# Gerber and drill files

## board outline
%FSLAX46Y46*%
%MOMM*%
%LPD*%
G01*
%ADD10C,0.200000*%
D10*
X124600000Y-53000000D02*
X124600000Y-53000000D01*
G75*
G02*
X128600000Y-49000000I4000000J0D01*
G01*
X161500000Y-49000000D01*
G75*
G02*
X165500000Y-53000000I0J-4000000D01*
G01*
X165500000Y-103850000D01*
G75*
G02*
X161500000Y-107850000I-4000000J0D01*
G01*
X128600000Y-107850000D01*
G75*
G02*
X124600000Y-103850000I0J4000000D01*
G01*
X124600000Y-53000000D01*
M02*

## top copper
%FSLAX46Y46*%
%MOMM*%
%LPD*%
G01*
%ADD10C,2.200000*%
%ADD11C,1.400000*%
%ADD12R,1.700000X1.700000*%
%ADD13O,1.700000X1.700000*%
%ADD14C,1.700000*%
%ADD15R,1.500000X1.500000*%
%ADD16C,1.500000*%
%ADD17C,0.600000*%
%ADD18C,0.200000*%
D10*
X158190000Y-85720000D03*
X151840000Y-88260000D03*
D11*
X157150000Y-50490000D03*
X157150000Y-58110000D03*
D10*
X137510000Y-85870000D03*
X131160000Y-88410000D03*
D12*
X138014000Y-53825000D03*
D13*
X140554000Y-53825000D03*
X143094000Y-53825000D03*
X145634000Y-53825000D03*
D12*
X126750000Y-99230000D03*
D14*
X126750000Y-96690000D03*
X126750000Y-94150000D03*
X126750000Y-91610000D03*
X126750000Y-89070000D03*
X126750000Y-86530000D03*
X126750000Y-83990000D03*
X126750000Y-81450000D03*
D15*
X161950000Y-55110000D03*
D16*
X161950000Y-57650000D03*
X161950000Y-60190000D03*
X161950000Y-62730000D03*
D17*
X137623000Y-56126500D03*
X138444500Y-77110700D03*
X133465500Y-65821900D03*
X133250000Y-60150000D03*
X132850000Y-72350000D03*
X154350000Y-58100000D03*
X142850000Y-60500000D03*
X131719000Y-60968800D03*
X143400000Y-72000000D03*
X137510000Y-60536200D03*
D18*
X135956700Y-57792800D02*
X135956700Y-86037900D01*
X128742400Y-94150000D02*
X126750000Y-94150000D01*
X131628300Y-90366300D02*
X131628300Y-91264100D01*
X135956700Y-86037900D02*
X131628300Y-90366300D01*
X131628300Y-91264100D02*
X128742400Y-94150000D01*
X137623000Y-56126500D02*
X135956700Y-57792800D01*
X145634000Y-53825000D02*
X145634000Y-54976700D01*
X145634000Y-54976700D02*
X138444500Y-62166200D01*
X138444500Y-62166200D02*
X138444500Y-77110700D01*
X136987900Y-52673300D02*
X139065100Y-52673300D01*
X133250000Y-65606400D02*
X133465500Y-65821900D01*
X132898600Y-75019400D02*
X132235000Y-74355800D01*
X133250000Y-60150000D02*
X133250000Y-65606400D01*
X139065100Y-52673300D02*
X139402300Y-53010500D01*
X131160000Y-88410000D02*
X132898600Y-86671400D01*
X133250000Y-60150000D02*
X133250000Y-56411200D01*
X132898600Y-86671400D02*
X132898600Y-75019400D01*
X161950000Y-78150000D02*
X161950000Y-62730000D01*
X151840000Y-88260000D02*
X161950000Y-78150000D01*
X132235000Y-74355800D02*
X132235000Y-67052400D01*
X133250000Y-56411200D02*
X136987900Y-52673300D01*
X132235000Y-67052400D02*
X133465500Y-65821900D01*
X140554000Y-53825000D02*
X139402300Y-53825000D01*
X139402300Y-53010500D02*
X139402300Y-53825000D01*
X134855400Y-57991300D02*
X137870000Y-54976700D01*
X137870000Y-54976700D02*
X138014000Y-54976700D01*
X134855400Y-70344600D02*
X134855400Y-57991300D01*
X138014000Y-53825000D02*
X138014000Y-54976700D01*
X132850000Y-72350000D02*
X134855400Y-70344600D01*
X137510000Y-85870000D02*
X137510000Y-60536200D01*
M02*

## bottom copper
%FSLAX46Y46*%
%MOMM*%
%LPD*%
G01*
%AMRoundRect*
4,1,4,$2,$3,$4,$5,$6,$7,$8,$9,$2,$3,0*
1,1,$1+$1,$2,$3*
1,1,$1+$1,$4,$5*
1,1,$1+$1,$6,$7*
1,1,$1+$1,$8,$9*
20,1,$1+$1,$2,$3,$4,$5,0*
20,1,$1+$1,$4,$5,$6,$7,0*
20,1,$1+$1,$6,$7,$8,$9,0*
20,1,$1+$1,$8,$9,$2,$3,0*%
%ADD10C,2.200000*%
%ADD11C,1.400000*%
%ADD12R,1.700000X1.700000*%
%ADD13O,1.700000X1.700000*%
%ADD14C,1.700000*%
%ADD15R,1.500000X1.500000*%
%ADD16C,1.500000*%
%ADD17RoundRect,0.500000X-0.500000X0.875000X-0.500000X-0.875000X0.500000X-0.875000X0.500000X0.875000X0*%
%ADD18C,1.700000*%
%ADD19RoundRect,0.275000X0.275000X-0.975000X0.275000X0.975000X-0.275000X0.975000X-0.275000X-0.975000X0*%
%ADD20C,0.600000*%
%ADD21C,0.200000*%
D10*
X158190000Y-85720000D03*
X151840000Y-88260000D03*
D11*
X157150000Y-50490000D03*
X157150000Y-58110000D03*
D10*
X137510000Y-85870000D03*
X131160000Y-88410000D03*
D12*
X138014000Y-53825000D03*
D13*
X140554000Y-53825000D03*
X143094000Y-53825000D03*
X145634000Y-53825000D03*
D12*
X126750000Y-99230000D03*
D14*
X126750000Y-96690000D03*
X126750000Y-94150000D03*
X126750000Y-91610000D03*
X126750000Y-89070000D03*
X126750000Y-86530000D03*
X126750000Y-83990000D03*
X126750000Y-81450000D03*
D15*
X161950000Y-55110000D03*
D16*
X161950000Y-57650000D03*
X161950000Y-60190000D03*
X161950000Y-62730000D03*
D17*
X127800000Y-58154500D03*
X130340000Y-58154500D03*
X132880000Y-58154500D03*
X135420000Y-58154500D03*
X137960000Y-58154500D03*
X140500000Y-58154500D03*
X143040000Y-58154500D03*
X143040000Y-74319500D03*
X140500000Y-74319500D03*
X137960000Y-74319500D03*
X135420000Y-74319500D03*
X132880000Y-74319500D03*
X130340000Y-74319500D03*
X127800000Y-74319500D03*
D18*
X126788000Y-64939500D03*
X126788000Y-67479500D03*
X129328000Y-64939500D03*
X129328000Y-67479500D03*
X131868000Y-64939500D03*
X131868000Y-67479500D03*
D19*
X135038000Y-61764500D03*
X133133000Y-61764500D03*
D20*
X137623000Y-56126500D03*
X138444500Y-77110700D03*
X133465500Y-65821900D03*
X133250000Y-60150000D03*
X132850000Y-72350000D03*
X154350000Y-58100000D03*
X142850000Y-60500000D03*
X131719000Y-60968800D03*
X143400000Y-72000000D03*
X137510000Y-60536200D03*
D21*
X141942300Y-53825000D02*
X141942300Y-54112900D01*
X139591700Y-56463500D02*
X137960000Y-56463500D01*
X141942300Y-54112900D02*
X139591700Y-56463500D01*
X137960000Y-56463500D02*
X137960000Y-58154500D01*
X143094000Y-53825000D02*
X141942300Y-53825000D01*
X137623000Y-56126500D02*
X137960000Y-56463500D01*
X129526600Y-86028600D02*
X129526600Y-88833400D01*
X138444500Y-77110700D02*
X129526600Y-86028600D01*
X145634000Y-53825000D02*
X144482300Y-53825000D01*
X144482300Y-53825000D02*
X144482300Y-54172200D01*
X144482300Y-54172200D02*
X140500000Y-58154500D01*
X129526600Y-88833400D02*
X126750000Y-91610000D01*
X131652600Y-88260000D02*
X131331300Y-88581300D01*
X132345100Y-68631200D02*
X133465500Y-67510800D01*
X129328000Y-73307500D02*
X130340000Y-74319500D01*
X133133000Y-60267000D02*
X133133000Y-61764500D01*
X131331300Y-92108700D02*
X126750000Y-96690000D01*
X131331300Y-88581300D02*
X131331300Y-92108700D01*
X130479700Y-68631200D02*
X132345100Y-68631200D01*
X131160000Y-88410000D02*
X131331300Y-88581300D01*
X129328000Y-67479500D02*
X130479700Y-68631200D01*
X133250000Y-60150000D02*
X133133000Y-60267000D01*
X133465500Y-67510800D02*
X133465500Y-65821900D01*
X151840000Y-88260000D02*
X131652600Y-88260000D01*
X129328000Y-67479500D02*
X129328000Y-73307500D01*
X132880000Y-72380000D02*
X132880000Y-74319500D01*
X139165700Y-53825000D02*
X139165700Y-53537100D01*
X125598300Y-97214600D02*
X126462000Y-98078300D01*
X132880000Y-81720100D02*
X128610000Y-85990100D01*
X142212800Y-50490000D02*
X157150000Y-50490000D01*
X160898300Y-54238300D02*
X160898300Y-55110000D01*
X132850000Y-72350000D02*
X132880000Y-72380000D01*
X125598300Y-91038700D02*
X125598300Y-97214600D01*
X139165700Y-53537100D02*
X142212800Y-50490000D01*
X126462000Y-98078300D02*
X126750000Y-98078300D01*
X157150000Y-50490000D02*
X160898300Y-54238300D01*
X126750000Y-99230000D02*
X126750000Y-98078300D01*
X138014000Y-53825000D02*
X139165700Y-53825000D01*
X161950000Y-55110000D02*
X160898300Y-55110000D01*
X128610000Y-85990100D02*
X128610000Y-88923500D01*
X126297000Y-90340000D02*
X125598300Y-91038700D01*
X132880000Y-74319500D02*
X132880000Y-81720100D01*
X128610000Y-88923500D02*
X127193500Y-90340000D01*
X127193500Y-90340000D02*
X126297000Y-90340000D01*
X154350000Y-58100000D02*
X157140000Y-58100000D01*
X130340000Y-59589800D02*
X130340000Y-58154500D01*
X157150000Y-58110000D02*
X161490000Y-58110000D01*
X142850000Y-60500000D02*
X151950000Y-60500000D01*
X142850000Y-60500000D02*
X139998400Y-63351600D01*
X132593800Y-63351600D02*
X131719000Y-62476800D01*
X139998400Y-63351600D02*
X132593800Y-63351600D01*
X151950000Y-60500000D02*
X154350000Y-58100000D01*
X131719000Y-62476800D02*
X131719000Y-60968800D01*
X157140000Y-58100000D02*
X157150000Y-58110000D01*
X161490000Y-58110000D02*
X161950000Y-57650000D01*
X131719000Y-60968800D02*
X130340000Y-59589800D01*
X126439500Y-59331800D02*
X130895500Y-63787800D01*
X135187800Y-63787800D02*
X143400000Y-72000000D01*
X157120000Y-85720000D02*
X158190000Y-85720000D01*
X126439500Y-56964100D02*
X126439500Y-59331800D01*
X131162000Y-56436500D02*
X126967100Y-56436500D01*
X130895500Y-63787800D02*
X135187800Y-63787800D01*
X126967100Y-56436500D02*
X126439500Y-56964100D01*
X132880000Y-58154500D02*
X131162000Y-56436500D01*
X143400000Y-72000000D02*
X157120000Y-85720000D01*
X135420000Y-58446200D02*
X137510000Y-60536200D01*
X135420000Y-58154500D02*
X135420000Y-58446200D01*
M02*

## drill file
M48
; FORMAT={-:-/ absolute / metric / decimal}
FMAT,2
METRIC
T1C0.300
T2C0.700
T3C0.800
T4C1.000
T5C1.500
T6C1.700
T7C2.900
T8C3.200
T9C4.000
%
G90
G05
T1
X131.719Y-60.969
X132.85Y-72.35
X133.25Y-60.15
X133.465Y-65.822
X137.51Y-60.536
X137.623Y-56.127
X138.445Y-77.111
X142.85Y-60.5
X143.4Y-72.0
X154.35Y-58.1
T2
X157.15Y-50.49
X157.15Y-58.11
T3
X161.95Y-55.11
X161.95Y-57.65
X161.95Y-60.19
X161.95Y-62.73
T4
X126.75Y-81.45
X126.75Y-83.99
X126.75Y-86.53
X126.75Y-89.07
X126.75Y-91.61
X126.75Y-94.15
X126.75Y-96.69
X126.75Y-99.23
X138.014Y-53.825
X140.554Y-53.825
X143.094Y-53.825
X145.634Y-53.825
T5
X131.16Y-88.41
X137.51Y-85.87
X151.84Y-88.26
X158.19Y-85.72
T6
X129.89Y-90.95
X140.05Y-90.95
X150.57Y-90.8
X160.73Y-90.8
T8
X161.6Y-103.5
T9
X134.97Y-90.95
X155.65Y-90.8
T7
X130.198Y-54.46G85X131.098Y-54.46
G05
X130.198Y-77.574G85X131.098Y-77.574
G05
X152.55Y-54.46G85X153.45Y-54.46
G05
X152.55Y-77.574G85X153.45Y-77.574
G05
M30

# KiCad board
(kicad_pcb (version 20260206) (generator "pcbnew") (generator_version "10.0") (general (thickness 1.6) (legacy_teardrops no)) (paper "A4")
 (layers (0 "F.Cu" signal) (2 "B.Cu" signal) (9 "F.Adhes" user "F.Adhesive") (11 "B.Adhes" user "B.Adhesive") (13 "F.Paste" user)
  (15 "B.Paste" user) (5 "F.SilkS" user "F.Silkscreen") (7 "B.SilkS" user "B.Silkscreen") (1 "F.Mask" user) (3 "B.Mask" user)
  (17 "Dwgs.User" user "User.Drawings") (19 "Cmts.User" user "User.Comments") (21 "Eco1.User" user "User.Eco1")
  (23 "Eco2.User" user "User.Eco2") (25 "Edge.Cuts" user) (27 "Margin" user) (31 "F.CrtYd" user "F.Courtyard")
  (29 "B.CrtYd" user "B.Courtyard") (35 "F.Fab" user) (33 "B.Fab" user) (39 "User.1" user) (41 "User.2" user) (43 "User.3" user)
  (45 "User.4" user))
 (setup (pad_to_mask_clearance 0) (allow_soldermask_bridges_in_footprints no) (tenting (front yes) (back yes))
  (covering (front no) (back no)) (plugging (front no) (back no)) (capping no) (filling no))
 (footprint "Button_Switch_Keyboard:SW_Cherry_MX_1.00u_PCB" (layer "F.Cu") (at 158.19 85.72)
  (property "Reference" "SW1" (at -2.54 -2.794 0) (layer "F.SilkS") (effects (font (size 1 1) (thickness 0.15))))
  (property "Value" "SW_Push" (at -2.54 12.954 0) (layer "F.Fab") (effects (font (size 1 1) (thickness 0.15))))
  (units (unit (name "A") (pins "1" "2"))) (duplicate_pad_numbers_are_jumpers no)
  (pad "" np_thru_hole circle (at -7.62 5.08) (size 1.7 1.7) (drill 1.7) (layers "*.Cu" "*.Mask"))
  (pad "" np_thru_hole circle (at -2.54 5.08) (size 4 4) (drill 4) (layers "*.Cu" "*.Mask"))
  (pad "" np_thru_hole circle (at 2.54 5.08) (size 1.7 1.7) (drill 1.7) (layers "*.Cu" "*.Mask"))
  (pad "1" thru_hole circle (at 0 0) (size 2.2 2.2) (drill 1.5) (layers "*.Cu" "*.Mask") (remove_unused_layers no) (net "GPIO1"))
  (pad "2" thru_hole circle (at -6.35 2.54) (size 2.2 2.2) (drill 1.5) (layers "*.Cu" "*.Mask") (remove_unused_layers no) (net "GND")))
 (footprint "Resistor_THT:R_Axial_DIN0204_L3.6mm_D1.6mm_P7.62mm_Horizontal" (layer "F.Cu") (at 157.15 50.49 -90)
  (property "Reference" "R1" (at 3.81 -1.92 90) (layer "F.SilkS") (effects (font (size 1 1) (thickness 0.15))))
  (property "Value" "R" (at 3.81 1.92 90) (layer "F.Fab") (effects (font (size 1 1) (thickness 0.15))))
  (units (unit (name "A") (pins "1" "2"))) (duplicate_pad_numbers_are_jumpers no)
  (pad "1" thru_hole circle (at 0 0 270) (size 1.4 1.4) (drill 0.7) (layers "*.Cu" "*.Mask") (remove_unused_layers no) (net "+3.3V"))
  (pad "2" thru_hole circle (at 7.62 0 270) (size 1.4 1.4) (drill 0.7) (layers "*.Cu" "*.Mask") (remove_unused_layers no) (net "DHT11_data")))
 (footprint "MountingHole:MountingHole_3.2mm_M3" (layer "F.Cu") (at 161.6 103.5)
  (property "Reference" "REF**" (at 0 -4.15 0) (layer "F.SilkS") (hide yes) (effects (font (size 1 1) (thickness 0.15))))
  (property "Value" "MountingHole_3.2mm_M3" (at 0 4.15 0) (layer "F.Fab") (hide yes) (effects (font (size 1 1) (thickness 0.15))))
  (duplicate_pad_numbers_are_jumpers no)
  (pad "" np_thru_hole circle (at 0 0) (size 3.2 3.2) (drill 3.2) (layers "*.Cu" "*.Mask")))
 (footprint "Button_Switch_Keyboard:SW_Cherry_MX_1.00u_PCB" (layer "F.Cu") (at 137.51 85.87)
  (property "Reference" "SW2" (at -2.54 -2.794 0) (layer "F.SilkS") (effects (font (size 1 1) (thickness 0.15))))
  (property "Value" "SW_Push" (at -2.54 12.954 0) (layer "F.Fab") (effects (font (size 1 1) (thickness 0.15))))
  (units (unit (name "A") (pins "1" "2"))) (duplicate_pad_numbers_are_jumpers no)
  (pad "" np_thru_hole circle (at -7.62 5.08) (size 1.7 1.7) (drill 1.7) (layers "*.Cu" "*.Mask"))
  (pad "" np_thru_hole circle (at -2.54 5.08) (size 4 4) (drill 4) (layers "*.Cu" "*.Mask"))
  (pad "" np_thru_hole circle (at 2.54 5.08) (size 1.7 1.7) (drill 1.7) (layers "*.Cu" "*.Mask"))
  (pad "1" thru_hole circle (at 0 0) (size 2.2 2.2) (drill 1.5) (layers "*.Cu" "*.Mask") (remove_unused_layers no) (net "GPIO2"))
  (pad "2" thru_hole circle (at -6.35 2.54) (size 2.2 2.2) (drill 1.5) (layers "*.Cu" "*.Mask") (remove_unused_layers no) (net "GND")))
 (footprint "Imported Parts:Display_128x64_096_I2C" (layer "F.Cu") (at 141.824 53.825)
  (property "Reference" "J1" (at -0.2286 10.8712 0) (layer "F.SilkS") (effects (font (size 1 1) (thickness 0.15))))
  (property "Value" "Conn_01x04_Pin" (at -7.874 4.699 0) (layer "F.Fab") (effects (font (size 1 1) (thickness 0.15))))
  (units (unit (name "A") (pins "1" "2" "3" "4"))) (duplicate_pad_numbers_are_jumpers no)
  (pad "" np_thru_hole oval (at -11.176 0.635) (size 3.8 2.9) (drill oval 3.8 2.9) (layers "*.Cu" "*.Mask"))
  (pad "" np_thru_hole oval (at -11.176 23.749) (size 3.8 2.9) (drill oval 3.8 2.9) (layers "*.Cu" "*.Mask"))
  (pad "" np_thru_hole oval (at 11.176 0.635) (size 3.8 2.9) (drill oval 3.8 2.9) (layers "*.Cu" "*.Mask"))
  (pad "" np_thru_hole oval (at 11.176 23.749) (size 3.8 2.9) (drill oval 3.8 2.9) (layers "*.Cu" "*.Mask"))
  (pad "1" thru_hole rect (at -3.81 0 90) (size 1.7 1.7) (drill 1) (layers "*.Cu" "*.Mask") (remove_unused_layers no) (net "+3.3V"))
  (pad "2" thru_hole oval (at -1.27 0 90) (size 1.7 1.7) (drill 1) (layers "*.Cu" "*.Mask") (remove_unused_layers no) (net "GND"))
  (pad "3" thru_hole oval (at 1.27 0 90) (size 1.7 1.7) (drill 1) (layers "*.Cu" "*.Mask") (remove_unused_layers no) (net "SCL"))
  (pad "4" thru_hole oval (at 3.81 0 90) (size 1.7 1.7) (drill 1) (layers "*.Cu" "*.Mask") (remove_unused_layers no) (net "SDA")))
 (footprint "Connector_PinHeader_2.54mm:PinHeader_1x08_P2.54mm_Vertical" (layer "B.Cu") (at 126.75 99.23)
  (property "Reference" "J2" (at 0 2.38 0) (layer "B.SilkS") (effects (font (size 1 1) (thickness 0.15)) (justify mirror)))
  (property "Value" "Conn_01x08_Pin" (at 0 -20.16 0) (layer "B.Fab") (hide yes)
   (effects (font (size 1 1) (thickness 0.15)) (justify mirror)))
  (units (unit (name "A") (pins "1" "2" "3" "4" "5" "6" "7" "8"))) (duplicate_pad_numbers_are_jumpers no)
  (pad "1" thru_hole rect (at 0 0) (size 1.7 1.7) (drill 1) (layers "*.Cu" "*.Mask") (remove_unused_layers no) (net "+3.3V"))
  (pad "2" thru_hole circle (at 0 -2.54) (size 1.7 1.7) (drill 1) (layers "*.Cu" "*.Mask") (remove_unused_layers no) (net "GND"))
  (pad "3" thru_hole circle (at 0 -5.08) (size 1.7 1.7) (drill 1) (layers "*.Cu" "*.Mask") (remove_unused_layers no) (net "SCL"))
  (pad "4" thru_hole circle (at 0 -7.62) (size 1.7 1.7) (drill 1) (layers "*.Cu" "*.Mask") (remove_unused_layers no) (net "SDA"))
  (pad "5" thru_hole circle (at 0 -10.16) (size 1.7 1.7) (drill 1) (layers "*.Cu" "*.Mask") (remove_unused_layers no)
   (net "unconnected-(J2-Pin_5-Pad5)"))
  (pad "6" thru_hole circle (at 0 -12.7) (size 1.7 1.7) (drill 1) (layers "*.Cu" "*.Mask") (remove_unused_layers no)
   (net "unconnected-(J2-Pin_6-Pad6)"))
  (pad "7" thru_hole circle (at 0 -15.24) (size 1.7 1.7) (drill 1) (layers "*.Cu" "*.Mask") (remove_unused_layers no)
   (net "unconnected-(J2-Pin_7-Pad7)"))
  (pad "8" thru_hole circle (at 0 -17.78) (size 1.7 1.7) (drill 1) (layers "*.Cu" "*.Mask") (remove_unused_layers no)
   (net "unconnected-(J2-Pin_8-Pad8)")))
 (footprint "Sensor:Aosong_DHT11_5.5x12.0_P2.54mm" (layer "B.Cu") (at 161.95 55.11 180)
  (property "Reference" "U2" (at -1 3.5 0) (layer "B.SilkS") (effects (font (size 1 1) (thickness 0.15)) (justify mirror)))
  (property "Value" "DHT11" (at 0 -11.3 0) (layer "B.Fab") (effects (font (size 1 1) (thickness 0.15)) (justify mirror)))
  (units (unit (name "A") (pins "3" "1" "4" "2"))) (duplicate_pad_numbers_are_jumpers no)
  (pad "1" thru_hole rect (at 0 0 180) (size 1.5 1.5) (drill 0.8) (layers "*.Cu" "*.Mask") (remove_unused_layers no) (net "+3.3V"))
  (pad "2" thru_hole circle (at 0 -2.54 180) (size 1.5 1.5) (drill 0.8) (layers "*.Cu" "*.Mask") (remove_unused_layers no)
   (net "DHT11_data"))
  (pad "3" thru_hole circle (at 0 -5.08 180) (size 1.5 1.5) (drill 0.8) (layers "*.Cu" "*.Mask") (remove_unused_layers no)
   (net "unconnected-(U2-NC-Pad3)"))
  (pad "4" thru_hole circle (at 0 -7.62 180) (size 1.5 1.5) (drill 0.8) (layers "*.Cu" "*.Mask") (remove_unused_layers no) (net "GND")))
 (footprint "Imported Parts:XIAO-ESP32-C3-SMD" (layer "B.Cu") (at 145.92 57.3195 -90)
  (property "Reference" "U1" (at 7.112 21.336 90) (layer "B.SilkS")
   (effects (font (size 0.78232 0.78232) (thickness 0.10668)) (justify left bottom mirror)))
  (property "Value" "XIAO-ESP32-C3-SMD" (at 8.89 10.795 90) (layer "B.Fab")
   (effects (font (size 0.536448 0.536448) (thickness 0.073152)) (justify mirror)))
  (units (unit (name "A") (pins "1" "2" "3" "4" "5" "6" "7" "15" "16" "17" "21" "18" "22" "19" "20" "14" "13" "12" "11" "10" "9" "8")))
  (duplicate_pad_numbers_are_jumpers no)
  (pad "1" smd roundrect (at 0.835 18.12 270) (size 2.75 2) (layers "B.Cu" "B.Mask" "B.Paste") (roundrect_rratio 0.25)
   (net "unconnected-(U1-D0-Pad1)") (solder_mask_margin 0.0508) (thermal_bridge_angle 45))
  (pad "2" smd roundrect (at 0.835 15.58 270) (size 2.75 2) (layers "B.Cu" "B.Mask" "B.Paste") (roundrect_rratio 0.25) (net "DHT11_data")
   (solder_mask_margin 0.0508) (thermal_bridge_angle 45))
  (pad "3" smd roundrect (at 0.835 13.04 270) (size 2.75 2) (layers "B.Cu" "B.Mask" "B.Paste") (roundrect_rratio 0.25) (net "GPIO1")
   (solder_mask_margin 0.0508) (thermal_bridge_angle 45))
  (pad "4" smd roundrect (at 0.835 10.5 270) (size 2.75 2) (layers "B.Cu" "B.Mask" "B.Paste") (roundrect_rratio 0.25) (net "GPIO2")
   (solder_mask_margin 0.0508) (thermal_bridge_angle 45))
  (pad "5" smd roundrect (at 0.835 7.96 270) (size 2.75 2) (layers "B.Cu" "B.Mask" "B.Paste") (roundrect_rratio 0.25) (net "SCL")
   (solder_mask_margin 0.0508) (thermal_bridge_angle 45))
  (pad "6" smd roundrect (at 0.835 5.42 270) (size 2.75 2) (layers "B.Cu" "B.Mask" "B.Paste") (roundrect_rratio 0.25) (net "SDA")
   (solder_mask_margin 0.0508) (thermal_bridge_angle 45))
  (pad "7" smd roundrect (at 0.835 2.88 270) (size 2.75 2) (layers "B.Cu" "B.Mask" "B.Paste") (roundrect_rratio 0.25)
   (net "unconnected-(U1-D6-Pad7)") (solder_mask_margin 0.0508) (thermal_bridge_angle 45))
  (pad "8" smd roundrect (at 17 2.88 270) (size 2.75 2) (layers "B.Cu" "B.Mask" "B.Paste") (roundrect_rratio 0.25)
   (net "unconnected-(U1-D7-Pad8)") (solder_mask_margin 0.0508) (thermal_bridge_angle 45))
  (pad "9" smd roundrect (at 17 5.42 270) (size 2.75 2) (layers "B.Cu" "B.Mask" "B.Paste") (roundrect_rratio 0.25)
   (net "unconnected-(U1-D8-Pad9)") (solder_mask_margin 0.0508) (thermal_bridge_angle 45))
  (pad "10" smd roundrect (at 17 7.96 270) (size 2.75 2) (layers "B.Cu" "B.Mask" "B.Paste") (roundrect_rratio 0.25)
   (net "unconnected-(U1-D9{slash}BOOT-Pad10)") (solder_mask_margin 0.0508) (thermal_bridge_angle 45))
  (pad "11" smd roundrect (at 17 10.5 270) (size 2.75 2) (layers "B.Cu" "B.Mask" "B.Paste") (roundrect_rratio 0.25)
   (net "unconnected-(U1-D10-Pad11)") (solder_mask_margin 0.0508) (thermal_bridge_angle 45))
  (pad "12" smd roundrect (at 17 13.04 270) (size 2.75 2) (layers "B.Cu" "B.Mask" "B.Paste") (roundrect_rratio 0.25) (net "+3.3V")
   (solder_mask_margin 0.0508) (thermal_bridge_angle 45))
  (pad "13" smd roundrect (at 17 15.58 270) (size 2.75 2) (layers "B.Cu" "B.Mask" "B.Paste") (roundrect_rratio 0.25) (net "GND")
   (solder_mask_margin 0.0508) (thermal_bridge_angle 45))
  (pad "14" smd roundrect (at 17 18.12 270) (size 2.75 2) (layers "B.Cu" "B.Mask" "B.Paste") (roundrect_rratio 0.25) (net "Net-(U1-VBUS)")
   (solder_mask_margin 0.0508) (thermal_bridge_angle 45))
  (pad "15" smd circle (at 7.62 19.132 270) (size 1.7 1.7) (layers "B.Cu" "B.Mask" "B.Paste") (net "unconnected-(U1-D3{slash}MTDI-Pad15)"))
  (pad "16" smd circle (at 10.16 19.132 270) (size 1.7 1.7) (layers "B.Cu" "B.Mask" "B.Paste") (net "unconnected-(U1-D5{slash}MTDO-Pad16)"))
  (pad "17" smd circle (at 7.62 16.592 270) (size 1.7 1.7) (layers "B.Cu" "B.Mask" "B.Paste") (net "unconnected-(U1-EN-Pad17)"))
  (pad "18" smd circle (at 10.16 16.592 270) (size 1.7 1.7) (layers "B.Cu" "B.Mask" "B.Paste") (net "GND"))
  (pad "19" smd circle (at 7.62 14.052 270) (size 1.7 1.7) (layers "B.Cu" "B.Mask" "B.Paste") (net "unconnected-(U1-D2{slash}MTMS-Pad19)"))
  (pad "20" smd circle (at 10.16 14.052 270) (size 1.7 1.7) (layers "B.Cu" "B.Mask" "B.Paste") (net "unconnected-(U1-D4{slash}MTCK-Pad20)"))
  (pad "21" smd roundrect (at 4.445 10.882 90) (size 2.5 1.1) (layers "B.Cu" "B.Mask" "B.Paste") (roundrect_rratio 0.25)
   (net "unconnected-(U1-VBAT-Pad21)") (thermal_bridge_angle 45))
  (pad "22" smd roundrect (at 4.445 12.787 90) (size 2.5 1.1) (layers "B.Cu" "B.Mask" "B.Paste") (roundrect_rratio 0.25) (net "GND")
   (thermal_bridge_angle 45)))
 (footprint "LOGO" (layer "B.Cu") (at 151.821269 66.65 180)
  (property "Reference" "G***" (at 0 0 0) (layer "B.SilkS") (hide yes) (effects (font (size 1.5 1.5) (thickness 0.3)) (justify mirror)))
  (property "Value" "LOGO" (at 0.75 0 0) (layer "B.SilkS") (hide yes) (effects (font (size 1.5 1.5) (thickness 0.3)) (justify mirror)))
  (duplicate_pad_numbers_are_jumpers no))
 (gr_rect (start 124.6 49) (end 165.5 107.85) (radius 4) (stroke (width 0.2) (type solid)) (fill no) (layer "Edge.Cuts"))
 (segment (start 135.9567 57.7928) (end 135.9567 86.0379) (width 0.2) (layer "F.Cu") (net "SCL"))
 (segment (start 128.7424 94.15) (end 126.75 94.15) (width 0.2) (layer "F.Cu") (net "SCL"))
 (segment (start 131.6283 90.3663) (end 131.6283 91.2641) (width 0.2) (layer "F.Cu") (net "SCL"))
 (segment (start 135.9567 86.0379) (end 131.6283 90.3663) (width 0.2) (layer "F.Cu") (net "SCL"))
 (segment (start 131.6283 91.2641) (end 128.7424 94.15) (width 0.2) (layer "F.Cu") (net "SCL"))
 (segment (start 137.623 56.1265) (end 135.9567 57.7928) (width 0.2) (layer "F.Cu") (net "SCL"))
 (via (at 137.623 56.1265) (size 0.6) (drill 0.3) (layers "F.Cu" "B.Cu") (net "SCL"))
 (segment (start 141.9423 53.825) (end 141.9423 54.1129) (width 0.2) (layer "B.Cu") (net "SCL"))
 (segment (start 139.5917 56.4635) (end 137.96 56.4635) (width 0.2) (layer "B.Cu") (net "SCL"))
 (segment (start 141.9423 54.1129) (end 139.5917 56.4635) (width 0.2) (layer "B.Cu") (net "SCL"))
 (segment (start 137.96 56.4635) (end 137.96 58.1545) (width 0.2) (layer "B.Cu") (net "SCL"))
 (segment (start 143.094 53.825) (end 141.9423 53.825) (width 0.2) (layer "B.Cu") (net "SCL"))
 (segment (start 137.623 56.1265) (end 137.96 56.4635) (width 0.2) (layer "B.Cu") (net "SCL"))
 (segment (start 145.634 53.825) (end 145.634 54.9767) (width 0.2) (layer "F.Cu") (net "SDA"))
 (segment (start 145.634 54.9767) (end 138.4445 62.1662) (width 0.2) (layer "F.Cu") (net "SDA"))
 (segment (start 138.4445 62.1662) (end 138.4445 77.1107) (width 0.2) (layer "F.Cu") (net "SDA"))
 (via (at 138.4445 77.1107) (size 0.6) (drill 0.3) (layers "F.Cu" "B.Cu") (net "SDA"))
 (segment (start 129.5266 86.0286) (end 129.5266 88.8334) (width 0.2) (layer "B.Cu") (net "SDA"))
 (segment (start 138.4445 77.1107) (end 129.5266 86.0286) (width 0.2) (layer "B.Cu") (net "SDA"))
 (segment (start 145.634 53.825) (end 144.4823 53.825) (width 0.2) (layer "B.Cu") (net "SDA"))
 (segment (start 144.4823 53.825) (end 144.4823 54.1722) (width 0.2) (layer "B.Cu") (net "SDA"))
 (segment (start 144.4823 54.1722) (end 140.5 58.1545) (width 0.2) (layer "B.Cu") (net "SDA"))
 (segment (start 129.5266 88.8334) (end 126.75 91.61) (width 0.2) (layer "B.Cu") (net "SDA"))
 (segment (start 136.9879 52.6733) (end 139.0651 52.6733) (width 0.2) (layer "F.Cu") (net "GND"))
 (segment (start 133.25 65.6064) (end 133.4655 65.8219) (width 0.2) (layer "F.Cu") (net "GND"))
 (segment (start 132.8986 75.0194) (end 132.235 74.3558) (width 0.2) (layer "F.Cu") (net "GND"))
 (segment (start 133.25 60.15) (end 133.25 65.6064) (width 0.2) (layer "F.Cu") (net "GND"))
 (segment (start 139.0651 52.6733) (end 139.4023 53.0105) (width 0.2) (layer "F.Cu") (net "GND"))
 (segment (start 131.16 88.41) (end 132.8986 86.6714) (width 0.2) (layer "F.Cu") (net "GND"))
 (segment (start 133.25 60.15) (end 133.25 56.4112) (width 0.2) (layer "F.Cu") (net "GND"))
 (segment (start 132.8986 86.6714) (end 132.8986 75.0194) (width 0.2) (layer "F.Cu") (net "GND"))
 (segment (start 161.95 78.15) (end 161.95 62.73) (width 0.2) (layer "F.Cu") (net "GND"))
 (segment (start 151.84 88.26) (end 161.95 78.15) (width 0.2) (layer "F.Cu") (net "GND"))
 (segment (start 132.235 74.3558) (end 132.235 67.0524) (width 0.2) (layer "F.Cu") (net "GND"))
 (segment (start 133.25 56.4112) (end 136.9879 52.6733) (width 0.2) (layer "F.Cu") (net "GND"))
 (segment (start 132.235 67.0524) (end 133.4655 65.8219) (width 0.2) (layer "F.Cu") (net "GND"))
 (segment (start 140.554 53.825) (end 139.4023 53.825) (width 0.2) (layer "F.Cu") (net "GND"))
 (segment (start 139.4023 53.0105) (end 139.4023 53.825) (width 0.2) (layer "F.Cu") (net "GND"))
 (via (at 133.4655 65.8219) (size 0.6) (drill 0.3) (layers "F.Cu" "B.Cu") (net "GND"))
 (via (at 133.25 60.15) (size 0.6) (drill 0.3) (layers "F.Cu" "B.Cu") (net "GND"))
 (segment (start 131.6526 88.26) (end 131.3313 88.5813) (width 0.2) (layer "B.Cu") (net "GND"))
 (segment (start 132.3451 68.6312) (end 133.4655 67.5108) (width 0.2) (layer "B.Cu") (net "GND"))
 (segment (start 129.328 73.3075) (end 130.34 74.3195) (width 0.2) (layer "B.Cu") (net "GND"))
 (segment (start 133.133 60.267) (end 133.133 61.7645) (width 0.2) (layer "B.Cu") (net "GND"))
 (segment (start 131.3313 92.1087) (end 126.75 96.69) (width 0.2) (layer "B.Cu") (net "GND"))
 (segment (start 131.3313 88.5813) (end 131.3313 92.1087) (width 0.2) (layer "B.Cu") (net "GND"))
 (segment (start 130.4797 68.6312) (end 132.3451 68.6312) (width 0.2) (layer "B.Cu") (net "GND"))
 (segment (start 131.16 88.41) (end 131.3313 88.5813) (width 0.2) (layer "B.Cu") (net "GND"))
 (segment (start 129.328 67.4795) (end 130.4797 68.6312) (width 0.2) (layer "B.Cu") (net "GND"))
 (segment (start 133.25 60.15) (end 133.133 60.267) (width 0.2) (layer "B.Cu") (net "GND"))
 (segment (start 133.4655 67.5108) (end 133.4655 65.8219) (width 0.2) (layer "B.Cu") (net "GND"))
 (segment (start 151.84 88.26) (end 131.6526 88.26) (width 0.2) (layer "B.Cu") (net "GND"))
 (segment (start 129.328 67.4795) (end 129.328 73.3075) (width 0.2) (layer "B.Cu") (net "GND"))
 (segment (start 134.8554 57.9913) (end 137.87 54.9767) (width 0.2) (layer "F.Cu") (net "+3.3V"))
 (segment (start 137.87 54.9767) (end 138.014 54.9767) (width 0.2) (layer "F.Cu") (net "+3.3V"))
 (segment (start 134.8554 70.3446) (end 134.8554 57.9913) (width 0.2) (layer "F.Cu") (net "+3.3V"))
 (segment (start 138.014 53.825) (end 138.014 54.9767) (width 0.2) (layer "F.Cu") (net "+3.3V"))
 (segment (start 132.85 72.35) (end 134.8554 70.3446) (width 0.2) (layer "F.Cu") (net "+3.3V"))
 (via (at 132.85 72.35) (size 0.6) (drill 0.3) (layers "F.Cu" "B.Cu") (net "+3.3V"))
 (segment (start 132.88 72.38) (end 132.88 74.3195) (width 0.2) (layer "B.Cu") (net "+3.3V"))
 (segment (start 139.1657 53.825) (end 139.1657 53.5371) (width 0.2) (layer "B.Cu") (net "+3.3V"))
 (segment (start 125.5983 97.2146) (end 126.462 98.0783) (width 0.2) (layer "B.Cu") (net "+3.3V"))
 (segment (start 132.88 81.7201) (end 128.61 85.9901) (width 0.2) (layer "B.Cu") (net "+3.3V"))
 (segment (start 142.2128 50.49) (end 157.15 50.49) (width 0.2) (layer "B.Cu") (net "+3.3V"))
 (segment (start 160.8983 54.2383) (end 160.8983 55.11) (width 0.2) (layer "B.Cu") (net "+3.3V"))
 (segment (start 132.85 72.35) (end 132.88 72.38) (width 0.2) (layer "B.Cu") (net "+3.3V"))
 (segment (start 125.5983 91.0387) (end 125.5983 97.2146) (width 0.2) (layer "B.Cu") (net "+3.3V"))
 (segment (start 139.1657 53.5371) (end 142.2128 50.49) (width 0.2) (layer "B.Cu") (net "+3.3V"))
 (segment (start 126.462 98.0783) (end 126.75 98.0783) (width 0.2) (layer "B.Cu") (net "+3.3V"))
 (segment (start 157.15 50.49) (end 160.8983 54.2383) (width 0.2) (layer "B.Cu") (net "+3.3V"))
 (segment (start 126.75 99.23) (end 126.75 98.0783) (width 0.2) (layer "B.Cu") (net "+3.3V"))
 (segment (start 138.014 53.825) (end 139.1657 53.825) (width 0.2) (layer "B.Cu") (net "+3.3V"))
 (segment (start 161.95 55.11) (end 160.8983 55.11) (width 0.2) (layer "B.Cu") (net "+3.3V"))
 (segment (start 128.61 85.9901) (end 128.61 88.9235) (width 0.2) (layer "B.Cu") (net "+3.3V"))
 (segment (start 126.297 90.34) (end 125.5983 91.0387) (width 0.2) (layer "B.Cu") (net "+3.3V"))
 (segment (start 132.88 74.3195) (end 132.88 81.7201) (width 0.2) (layer "B.Cu") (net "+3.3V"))
 (segment (start 128.61 88.9235) (end 127.1935 90.34) (width 0.2) (layer "B.Cu") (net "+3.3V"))
 (segment (start 127.1935 90.34) (end 126.297 90.34) (width 0.2) (layer "B.Cu") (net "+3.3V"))
 (via (at 154.35 58.1) (size 0.6) (drill 0.3) (layers "F.Cu" "B.Cu") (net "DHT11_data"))
 (via (at 142.85 60.5) (size 0.6) (drill 0.3) (layers "F.Cu" "B.Cu") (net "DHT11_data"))
 (via (at 131.719 60.9688) (size 0.6) (drill 0.3) (layers "F.Cu" "B.Cu") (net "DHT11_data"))
 (segment (start 154.35 58.1) (end 157.14 58.1) (width 0.2) (layer "B.Cu") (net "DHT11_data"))
 (segment (start 130.34 59.5898) (end 130.34 58.1545) (width 0.2) (layer "B.Cu") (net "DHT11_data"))
 (segment (start 157.15 58.11) (end 161.49 58.11) (width 0.2) (layer "B.Cu") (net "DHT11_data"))
 (segment (start 142.85 60.5) (end 151.95 60.5) (width 0.2) (layer "B.Cu") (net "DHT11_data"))
 (segment (start 142.85 60.5) (end 139.9984 63.3516) (width 0.2) (layer "B.Cu") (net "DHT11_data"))
 (segment (start 132.5938 63.3516) (end 131.719 62.4768) (width 0.2) (layer "B.Cu") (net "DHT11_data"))
 (segment (start 139.9984 63.3516) (end 132.5938 63.3516) (width 0.2) (layer "B.Cu") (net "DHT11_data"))
 (segment (start 151.95 60.5) (end 154.35 58.1) (width 0.2) (layer "B.Cu") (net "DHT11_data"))
 (segment (start 131.719 62.4768) (end 131.719 60.9688) (width 0.2) (layer "B.Cu") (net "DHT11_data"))
 (segment (start 157.14 58.1) (end 157.15 58.11) (width 0.2) (layer "B.Cu") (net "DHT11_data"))
 (segment (start 161.49 58.11) (end 161.95 57.65) (width 0.2) (layer "B.Cu") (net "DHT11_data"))
 (segment (start 131.719 60.9688) (end 130.34 59.5898) (width 0.2) (layer "B.Cu") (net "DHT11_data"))
 (via (at 143.4 72) (size 0.6) (drill 0.3) (layers "F.Cu" "B.Cu") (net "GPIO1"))
 (segment (start 126.4395 59.3318) (end 130.8955 63.7878) (width 0.2) (layer "B.Cu") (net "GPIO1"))
 (segment (start 135.1878 63.7878) (end 143.4 72) (width 0.2) (layer "B.Cu") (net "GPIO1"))
 (segment (start 157.12 85.72) (end 158.19 85.72) (width 0.2) (layer "B.Cu") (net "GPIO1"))
 (segment (start 126.4395 56.9641) (end 126.4395 59.3318) (width 0.2) (layer "B.Cu") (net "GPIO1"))
 (segment (start 131.162 56.4365) (end 126.9671 56.4365) (width 0.2) (layer "B.Cu") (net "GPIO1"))
 (segment (start 130.8955 63.7878) (end 135.1878 63.7878) (width 0.2) (layer "B.Cu") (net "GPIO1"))
 (segment (start 126.9671 56.4365) (end 126.4395 56.9641) (width 0.2) (layer "B.Cu") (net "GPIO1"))
 (segment (start 132.88 58.1545) (end 131.162 56.4365) (width 0.2) (layer "B.Cu") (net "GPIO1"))
 (segment (start 143.4 72) (end 157.12 85.72) (width 0.2) (layer "B.Cu") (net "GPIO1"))
 (segment (start 137.51 85.87) (end 137.51 60.5362) (width 0.2) (layer "F.Cu") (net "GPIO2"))
 (via (at 137.51 60.5362) (size 0.6) (drill 0.3) (layers "F.Cu" "B.Cu") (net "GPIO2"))
 (segment (start 135.42 58.4462) (end 137.51 60.5362) (width 0.2) (layer "B.Cu") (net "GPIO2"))
 (segment (start 135.42 58.1545) (end 135.42 58.4462) (width 0.2) (layer "B.Cu") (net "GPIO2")))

